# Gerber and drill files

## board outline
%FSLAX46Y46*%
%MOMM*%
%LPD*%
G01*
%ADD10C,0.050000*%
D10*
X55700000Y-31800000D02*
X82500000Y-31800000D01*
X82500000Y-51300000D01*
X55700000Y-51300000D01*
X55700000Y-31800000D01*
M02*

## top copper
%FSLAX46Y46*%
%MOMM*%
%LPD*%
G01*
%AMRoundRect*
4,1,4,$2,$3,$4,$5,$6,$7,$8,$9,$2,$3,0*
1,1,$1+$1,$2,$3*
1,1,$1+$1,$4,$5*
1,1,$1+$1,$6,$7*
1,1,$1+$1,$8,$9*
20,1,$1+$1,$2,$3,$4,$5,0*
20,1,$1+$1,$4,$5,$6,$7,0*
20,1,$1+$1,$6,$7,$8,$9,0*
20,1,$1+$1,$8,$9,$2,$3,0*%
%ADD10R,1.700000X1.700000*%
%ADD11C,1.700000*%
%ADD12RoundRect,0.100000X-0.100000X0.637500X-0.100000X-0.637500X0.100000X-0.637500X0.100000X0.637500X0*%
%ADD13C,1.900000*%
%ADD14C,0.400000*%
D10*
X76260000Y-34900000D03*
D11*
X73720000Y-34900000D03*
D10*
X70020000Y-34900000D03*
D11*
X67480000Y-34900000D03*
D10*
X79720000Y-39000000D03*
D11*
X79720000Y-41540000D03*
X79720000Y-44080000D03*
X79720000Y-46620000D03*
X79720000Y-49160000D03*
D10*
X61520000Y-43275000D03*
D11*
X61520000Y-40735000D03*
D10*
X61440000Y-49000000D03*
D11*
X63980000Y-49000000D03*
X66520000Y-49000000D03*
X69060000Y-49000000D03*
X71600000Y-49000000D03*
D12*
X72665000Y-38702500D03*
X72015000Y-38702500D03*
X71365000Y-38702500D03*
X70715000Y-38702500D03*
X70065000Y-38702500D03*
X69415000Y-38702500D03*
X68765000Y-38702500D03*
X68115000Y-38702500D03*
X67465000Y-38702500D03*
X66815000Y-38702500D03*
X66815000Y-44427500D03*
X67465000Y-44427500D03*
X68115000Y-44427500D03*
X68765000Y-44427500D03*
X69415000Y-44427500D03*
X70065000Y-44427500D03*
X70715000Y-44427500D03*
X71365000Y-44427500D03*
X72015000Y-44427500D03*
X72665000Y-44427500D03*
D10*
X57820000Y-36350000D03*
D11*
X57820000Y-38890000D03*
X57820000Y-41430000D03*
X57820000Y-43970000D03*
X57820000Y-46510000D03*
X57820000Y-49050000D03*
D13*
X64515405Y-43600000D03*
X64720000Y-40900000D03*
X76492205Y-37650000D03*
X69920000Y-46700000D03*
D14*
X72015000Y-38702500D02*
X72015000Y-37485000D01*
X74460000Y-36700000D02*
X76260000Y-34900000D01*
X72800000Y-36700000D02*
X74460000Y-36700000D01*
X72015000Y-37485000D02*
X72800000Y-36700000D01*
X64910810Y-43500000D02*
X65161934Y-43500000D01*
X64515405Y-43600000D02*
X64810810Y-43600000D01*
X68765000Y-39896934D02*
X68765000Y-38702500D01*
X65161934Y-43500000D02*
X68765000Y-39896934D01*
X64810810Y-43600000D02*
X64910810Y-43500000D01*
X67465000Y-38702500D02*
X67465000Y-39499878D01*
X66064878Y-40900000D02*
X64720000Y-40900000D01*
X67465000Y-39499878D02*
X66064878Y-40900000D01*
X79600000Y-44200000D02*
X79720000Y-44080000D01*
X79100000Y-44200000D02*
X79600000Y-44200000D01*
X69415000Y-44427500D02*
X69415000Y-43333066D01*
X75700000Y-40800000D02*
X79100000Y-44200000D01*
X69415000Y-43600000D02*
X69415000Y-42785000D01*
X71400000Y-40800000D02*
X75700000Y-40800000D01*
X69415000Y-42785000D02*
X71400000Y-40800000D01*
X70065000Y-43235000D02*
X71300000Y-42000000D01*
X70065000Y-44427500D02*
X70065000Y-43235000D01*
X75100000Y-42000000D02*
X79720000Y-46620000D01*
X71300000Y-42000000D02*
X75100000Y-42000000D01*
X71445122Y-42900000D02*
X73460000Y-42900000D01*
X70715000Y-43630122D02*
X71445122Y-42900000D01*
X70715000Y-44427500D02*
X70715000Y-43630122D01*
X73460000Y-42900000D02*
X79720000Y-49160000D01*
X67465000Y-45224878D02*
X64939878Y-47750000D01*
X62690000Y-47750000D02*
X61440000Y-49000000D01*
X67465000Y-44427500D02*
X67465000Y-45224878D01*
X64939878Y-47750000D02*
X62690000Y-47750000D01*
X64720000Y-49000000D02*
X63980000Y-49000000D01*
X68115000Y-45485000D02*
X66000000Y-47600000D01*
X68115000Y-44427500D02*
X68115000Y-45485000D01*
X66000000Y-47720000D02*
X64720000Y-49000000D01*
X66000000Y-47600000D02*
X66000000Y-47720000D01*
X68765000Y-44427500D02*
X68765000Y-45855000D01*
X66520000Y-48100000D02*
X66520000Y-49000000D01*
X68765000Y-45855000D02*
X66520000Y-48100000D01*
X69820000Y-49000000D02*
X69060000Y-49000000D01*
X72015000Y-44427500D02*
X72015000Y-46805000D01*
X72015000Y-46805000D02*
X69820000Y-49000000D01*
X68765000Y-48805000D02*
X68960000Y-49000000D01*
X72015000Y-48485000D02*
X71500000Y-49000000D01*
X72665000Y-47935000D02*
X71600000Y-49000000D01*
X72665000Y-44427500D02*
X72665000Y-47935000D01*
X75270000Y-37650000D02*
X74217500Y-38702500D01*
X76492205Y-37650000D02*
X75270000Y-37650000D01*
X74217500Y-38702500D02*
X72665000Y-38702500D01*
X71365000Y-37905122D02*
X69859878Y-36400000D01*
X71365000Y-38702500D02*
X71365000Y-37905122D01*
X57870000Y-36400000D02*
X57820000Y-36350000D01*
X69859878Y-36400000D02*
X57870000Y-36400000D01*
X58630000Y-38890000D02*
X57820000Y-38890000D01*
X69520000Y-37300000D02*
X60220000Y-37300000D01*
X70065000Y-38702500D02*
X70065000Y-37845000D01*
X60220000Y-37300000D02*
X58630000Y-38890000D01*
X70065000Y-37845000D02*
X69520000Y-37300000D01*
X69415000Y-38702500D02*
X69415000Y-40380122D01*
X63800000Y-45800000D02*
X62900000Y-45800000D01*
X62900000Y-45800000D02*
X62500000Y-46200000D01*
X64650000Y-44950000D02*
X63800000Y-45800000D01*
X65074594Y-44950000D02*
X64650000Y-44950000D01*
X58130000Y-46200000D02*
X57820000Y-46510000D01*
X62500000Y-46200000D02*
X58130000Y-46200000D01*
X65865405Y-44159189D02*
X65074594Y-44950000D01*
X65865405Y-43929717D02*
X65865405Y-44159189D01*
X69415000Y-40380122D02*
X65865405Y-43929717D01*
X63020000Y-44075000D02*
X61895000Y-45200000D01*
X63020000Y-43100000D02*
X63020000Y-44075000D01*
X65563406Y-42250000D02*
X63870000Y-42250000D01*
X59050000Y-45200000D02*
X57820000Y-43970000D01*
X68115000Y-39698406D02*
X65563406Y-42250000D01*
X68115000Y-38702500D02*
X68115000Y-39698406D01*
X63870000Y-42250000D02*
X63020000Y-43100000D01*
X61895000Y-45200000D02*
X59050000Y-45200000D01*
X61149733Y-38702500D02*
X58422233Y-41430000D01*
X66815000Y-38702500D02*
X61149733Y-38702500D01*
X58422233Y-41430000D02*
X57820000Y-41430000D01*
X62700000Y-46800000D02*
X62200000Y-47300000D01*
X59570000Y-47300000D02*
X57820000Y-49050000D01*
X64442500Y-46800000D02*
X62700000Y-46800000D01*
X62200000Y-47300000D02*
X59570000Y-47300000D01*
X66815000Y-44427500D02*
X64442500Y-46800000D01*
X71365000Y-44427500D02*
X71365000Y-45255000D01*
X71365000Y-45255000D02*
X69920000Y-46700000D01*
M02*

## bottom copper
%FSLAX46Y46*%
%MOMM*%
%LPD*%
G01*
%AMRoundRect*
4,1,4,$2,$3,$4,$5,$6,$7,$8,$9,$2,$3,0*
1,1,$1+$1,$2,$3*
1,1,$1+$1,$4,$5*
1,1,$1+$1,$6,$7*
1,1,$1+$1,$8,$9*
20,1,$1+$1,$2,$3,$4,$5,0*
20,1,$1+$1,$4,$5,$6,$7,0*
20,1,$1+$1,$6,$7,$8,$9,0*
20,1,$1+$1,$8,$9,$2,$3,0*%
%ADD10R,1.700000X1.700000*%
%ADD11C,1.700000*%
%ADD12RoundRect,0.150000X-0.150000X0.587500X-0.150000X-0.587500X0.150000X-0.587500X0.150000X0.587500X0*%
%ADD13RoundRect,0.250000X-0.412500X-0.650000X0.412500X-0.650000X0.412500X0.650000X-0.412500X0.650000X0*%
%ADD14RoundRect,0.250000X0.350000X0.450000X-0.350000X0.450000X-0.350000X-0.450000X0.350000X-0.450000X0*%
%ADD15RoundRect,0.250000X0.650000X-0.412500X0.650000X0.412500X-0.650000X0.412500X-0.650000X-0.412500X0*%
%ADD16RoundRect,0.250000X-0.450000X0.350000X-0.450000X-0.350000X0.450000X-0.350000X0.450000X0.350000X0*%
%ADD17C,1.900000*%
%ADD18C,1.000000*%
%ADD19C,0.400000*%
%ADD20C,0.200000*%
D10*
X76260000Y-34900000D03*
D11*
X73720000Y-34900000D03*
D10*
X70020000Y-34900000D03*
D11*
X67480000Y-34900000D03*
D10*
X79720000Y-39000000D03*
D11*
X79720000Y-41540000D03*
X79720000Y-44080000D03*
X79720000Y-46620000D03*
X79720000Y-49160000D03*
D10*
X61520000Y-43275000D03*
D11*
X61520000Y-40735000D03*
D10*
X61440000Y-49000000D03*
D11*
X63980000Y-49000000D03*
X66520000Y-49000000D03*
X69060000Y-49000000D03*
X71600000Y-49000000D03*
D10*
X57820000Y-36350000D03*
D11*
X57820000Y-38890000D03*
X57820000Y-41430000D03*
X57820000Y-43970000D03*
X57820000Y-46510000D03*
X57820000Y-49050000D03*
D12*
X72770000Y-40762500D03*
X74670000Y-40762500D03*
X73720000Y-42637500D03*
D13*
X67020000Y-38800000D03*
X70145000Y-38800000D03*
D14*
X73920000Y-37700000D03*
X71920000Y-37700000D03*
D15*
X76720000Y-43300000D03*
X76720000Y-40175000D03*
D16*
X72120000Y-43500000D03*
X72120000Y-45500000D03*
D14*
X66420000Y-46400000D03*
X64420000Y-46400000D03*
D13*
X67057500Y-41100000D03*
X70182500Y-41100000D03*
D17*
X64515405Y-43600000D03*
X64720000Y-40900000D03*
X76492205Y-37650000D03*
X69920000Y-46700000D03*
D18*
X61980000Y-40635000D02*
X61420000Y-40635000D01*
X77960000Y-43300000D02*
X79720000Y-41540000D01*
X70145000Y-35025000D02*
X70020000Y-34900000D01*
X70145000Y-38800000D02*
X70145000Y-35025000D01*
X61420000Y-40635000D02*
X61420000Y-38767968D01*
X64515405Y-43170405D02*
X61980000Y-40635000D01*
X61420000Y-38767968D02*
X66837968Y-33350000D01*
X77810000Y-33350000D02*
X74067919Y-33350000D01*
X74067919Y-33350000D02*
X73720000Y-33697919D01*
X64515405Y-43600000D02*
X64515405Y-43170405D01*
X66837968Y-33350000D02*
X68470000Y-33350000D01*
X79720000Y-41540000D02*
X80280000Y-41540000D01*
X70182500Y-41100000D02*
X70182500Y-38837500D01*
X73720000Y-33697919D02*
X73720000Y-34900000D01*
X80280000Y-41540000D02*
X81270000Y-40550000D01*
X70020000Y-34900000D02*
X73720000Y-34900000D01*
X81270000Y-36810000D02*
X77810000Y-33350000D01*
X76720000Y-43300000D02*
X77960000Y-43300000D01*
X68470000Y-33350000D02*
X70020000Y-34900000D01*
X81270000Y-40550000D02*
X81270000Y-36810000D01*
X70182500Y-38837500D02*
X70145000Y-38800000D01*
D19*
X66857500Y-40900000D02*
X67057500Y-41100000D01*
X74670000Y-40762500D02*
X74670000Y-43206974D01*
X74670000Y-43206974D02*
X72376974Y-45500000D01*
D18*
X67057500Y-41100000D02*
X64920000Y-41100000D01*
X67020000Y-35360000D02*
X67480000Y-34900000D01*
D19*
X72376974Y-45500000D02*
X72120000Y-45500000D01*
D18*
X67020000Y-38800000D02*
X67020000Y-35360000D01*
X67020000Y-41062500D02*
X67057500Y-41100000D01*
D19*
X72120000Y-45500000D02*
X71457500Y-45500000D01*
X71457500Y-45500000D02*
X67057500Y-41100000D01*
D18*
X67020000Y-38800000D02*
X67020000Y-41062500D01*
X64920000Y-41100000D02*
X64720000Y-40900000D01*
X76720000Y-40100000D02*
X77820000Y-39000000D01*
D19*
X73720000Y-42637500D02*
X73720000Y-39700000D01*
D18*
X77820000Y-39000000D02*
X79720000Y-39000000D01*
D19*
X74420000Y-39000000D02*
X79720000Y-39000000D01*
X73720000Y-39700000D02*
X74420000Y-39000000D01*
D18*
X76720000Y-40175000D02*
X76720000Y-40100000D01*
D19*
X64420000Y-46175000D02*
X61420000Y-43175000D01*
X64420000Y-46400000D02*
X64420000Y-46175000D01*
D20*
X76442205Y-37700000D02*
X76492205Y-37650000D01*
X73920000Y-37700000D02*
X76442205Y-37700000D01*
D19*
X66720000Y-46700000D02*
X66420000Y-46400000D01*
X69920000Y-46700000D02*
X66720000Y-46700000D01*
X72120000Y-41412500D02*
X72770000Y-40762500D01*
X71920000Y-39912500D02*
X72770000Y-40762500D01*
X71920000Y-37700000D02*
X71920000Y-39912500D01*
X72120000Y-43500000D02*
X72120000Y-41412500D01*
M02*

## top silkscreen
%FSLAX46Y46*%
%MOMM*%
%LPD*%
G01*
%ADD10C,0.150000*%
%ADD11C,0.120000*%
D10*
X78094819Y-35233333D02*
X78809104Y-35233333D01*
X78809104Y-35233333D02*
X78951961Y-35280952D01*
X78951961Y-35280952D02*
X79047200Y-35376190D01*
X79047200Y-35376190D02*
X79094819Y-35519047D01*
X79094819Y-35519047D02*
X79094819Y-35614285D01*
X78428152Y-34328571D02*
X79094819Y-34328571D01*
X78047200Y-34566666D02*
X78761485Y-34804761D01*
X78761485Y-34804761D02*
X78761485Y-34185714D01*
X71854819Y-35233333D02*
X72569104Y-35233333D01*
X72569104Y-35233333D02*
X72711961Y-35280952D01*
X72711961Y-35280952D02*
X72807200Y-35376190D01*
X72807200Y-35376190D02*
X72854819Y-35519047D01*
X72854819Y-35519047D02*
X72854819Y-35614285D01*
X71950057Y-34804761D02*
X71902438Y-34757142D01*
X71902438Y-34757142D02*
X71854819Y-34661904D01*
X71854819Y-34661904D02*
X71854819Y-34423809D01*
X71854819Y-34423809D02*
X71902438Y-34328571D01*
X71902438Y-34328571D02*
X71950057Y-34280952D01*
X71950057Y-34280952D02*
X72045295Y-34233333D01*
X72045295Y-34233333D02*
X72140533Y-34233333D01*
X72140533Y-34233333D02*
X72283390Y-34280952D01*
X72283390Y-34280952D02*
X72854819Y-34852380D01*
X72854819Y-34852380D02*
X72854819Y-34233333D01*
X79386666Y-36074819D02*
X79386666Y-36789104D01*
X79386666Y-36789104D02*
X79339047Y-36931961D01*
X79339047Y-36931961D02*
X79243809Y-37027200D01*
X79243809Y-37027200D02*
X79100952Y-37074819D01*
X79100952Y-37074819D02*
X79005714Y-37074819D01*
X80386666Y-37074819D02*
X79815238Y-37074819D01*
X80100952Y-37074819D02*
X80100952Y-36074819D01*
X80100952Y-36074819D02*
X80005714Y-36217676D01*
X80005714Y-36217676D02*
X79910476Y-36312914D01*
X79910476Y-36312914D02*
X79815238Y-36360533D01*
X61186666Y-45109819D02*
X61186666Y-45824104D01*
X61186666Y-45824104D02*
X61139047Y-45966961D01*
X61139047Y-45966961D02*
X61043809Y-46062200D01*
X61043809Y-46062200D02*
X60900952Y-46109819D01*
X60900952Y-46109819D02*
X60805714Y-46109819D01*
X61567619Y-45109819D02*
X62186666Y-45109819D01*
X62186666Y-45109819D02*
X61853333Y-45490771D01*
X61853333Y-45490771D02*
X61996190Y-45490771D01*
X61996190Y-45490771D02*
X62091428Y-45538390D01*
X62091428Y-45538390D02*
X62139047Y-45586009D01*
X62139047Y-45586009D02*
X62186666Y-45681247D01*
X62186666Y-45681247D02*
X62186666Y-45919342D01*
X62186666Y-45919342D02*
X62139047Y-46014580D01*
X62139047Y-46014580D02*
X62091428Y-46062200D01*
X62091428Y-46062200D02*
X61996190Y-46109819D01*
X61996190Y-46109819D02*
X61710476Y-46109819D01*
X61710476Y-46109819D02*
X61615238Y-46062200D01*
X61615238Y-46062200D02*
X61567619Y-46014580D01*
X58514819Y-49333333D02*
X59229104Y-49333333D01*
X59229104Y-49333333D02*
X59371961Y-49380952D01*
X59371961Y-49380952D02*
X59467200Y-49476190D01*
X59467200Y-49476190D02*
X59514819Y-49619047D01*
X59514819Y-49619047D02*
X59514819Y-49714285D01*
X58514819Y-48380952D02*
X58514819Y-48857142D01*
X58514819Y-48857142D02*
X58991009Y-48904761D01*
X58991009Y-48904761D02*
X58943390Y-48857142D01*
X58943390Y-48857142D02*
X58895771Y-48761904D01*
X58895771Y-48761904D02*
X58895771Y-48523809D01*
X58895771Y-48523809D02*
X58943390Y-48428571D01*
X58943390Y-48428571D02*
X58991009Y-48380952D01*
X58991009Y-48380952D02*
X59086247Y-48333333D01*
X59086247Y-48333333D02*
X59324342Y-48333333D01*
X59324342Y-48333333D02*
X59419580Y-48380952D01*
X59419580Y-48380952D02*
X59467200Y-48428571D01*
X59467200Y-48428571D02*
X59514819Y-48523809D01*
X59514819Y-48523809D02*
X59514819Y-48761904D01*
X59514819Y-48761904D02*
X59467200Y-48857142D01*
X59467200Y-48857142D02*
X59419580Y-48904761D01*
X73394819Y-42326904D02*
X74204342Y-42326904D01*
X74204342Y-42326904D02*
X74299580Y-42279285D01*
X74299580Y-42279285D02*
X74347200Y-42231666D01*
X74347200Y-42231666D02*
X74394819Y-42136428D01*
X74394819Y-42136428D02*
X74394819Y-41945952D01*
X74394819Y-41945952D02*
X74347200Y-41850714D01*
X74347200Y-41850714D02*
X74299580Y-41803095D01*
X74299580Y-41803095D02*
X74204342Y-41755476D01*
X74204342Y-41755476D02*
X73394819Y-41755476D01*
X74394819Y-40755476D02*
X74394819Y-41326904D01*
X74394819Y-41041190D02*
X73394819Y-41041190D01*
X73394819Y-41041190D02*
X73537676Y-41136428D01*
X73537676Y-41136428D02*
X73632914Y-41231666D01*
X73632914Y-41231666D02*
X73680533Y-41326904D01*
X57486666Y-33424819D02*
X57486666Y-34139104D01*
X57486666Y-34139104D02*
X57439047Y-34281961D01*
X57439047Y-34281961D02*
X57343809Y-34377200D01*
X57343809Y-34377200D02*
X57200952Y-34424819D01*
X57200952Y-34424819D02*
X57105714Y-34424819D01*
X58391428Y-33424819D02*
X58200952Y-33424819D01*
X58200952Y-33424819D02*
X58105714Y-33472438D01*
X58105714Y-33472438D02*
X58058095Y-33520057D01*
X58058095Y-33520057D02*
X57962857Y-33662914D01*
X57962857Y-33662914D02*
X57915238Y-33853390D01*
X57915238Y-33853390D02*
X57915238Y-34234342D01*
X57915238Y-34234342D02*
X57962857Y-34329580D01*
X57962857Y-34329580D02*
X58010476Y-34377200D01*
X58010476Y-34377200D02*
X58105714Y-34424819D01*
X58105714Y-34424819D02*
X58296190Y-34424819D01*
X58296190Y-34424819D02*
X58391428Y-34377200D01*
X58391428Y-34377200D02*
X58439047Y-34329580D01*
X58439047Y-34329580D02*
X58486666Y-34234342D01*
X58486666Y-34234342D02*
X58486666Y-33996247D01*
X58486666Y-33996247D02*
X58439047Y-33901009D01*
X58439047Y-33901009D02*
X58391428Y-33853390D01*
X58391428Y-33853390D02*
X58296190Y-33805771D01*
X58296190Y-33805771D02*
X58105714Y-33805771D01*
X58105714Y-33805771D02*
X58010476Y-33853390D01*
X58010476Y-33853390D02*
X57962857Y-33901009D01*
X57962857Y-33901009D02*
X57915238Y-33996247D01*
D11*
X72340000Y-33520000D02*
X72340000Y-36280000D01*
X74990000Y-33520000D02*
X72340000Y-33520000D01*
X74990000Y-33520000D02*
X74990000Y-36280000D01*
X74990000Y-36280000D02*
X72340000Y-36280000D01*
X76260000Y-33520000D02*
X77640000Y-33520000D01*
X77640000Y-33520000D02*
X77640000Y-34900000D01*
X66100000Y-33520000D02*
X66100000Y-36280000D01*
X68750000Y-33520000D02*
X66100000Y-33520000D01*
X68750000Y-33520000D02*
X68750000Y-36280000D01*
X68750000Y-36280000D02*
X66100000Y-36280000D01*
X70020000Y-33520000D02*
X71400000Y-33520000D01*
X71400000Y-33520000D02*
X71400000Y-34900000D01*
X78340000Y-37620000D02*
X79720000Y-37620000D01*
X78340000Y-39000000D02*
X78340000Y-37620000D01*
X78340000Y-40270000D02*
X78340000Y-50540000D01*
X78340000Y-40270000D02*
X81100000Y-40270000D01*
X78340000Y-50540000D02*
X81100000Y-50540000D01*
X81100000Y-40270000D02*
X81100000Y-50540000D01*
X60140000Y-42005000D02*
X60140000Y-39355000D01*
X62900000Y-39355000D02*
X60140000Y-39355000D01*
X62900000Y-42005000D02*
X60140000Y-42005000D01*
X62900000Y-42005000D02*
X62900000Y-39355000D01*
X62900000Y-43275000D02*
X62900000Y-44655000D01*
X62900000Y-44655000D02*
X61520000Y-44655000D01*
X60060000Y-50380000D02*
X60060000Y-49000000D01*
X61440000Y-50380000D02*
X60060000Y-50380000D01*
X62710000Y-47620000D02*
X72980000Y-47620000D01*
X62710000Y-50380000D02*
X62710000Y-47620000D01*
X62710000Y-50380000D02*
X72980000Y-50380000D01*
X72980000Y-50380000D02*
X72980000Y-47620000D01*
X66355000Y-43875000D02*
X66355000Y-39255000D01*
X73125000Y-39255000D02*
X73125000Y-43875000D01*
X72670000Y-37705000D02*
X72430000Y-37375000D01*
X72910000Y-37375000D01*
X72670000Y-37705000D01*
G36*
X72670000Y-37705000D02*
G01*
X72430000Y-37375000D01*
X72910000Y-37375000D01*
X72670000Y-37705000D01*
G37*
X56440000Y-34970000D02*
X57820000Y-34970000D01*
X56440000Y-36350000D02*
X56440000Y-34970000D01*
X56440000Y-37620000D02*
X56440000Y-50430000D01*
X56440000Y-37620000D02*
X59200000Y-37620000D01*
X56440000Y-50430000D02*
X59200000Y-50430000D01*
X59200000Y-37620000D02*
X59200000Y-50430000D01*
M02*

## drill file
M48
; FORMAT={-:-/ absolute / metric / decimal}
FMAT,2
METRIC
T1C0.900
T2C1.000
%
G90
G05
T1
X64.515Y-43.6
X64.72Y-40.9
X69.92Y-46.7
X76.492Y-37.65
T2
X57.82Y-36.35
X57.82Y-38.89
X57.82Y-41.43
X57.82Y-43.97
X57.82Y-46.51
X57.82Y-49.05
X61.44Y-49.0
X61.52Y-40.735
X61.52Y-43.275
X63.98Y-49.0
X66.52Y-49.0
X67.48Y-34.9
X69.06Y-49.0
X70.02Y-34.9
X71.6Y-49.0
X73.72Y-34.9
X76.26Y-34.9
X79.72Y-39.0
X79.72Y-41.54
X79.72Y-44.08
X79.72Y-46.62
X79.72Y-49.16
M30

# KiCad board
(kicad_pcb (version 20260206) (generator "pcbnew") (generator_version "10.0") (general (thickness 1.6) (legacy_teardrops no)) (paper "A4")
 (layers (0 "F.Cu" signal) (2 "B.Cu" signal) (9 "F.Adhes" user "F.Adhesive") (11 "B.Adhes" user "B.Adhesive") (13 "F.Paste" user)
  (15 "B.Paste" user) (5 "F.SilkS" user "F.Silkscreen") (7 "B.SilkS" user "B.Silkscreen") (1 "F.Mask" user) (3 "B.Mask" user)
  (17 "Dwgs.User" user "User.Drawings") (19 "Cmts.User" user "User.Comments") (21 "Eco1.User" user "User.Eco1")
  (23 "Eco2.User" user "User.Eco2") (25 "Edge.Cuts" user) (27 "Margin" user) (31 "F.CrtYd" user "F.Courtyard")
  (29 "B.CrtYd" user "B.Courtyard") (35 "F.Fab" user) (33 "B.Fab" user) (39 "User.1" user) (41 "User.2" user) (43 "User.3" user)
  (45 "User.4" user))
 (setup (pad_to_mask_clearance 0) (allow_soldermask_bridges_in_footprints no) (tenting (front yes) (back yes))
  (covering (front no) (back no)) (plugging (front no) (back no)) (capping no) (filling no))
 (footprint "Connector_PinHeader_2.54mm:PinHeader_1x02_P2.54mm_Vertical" (layer "F.Cu") (at 76.26 34.9 -90)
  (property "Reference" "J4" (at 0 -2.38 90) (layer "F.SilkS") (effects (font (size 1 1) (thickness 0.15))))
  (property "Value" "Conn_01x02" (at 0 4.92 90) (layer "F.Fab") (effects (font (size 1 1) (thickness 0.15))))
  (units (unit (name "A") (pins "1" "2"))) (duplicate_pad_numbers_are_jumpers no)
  (fp_line (start -1.38 3.92) (end 1.38 3.92) (stroke (width 0.12) (type solid)) (layer "F.SilkS"))
  (fp_line (start -1.38 1.27) (end -1.38 3.92) (stroke (width 0.12) (type solid)) (layer "F.SilkS"))
  (fp_line (start -1.38 1.27) (end 1.38 1.27) (stroke (width 0.12) (type solid)) (layer "F.SilkS"))
  (fp_line (start 1.38 1.27) (end 1.38 3.92) (stroke (width 0.12) (type solid)) (layer "F.SilkS"))
  (fp_line (start -1.38 0) (end -1.38 -1.38) (stroke (width 0.12) (type solid)) (layer "F.SilkS"))
  (fp_line (start -1.38 -1.38) (end 0 -1.38) (stroke (width 0.12) (type solid)) (layer "F.SilkS"))
  (pad "1" thru_hole rect (at 0 0 270) (size 1.7 1.7) (drill 1) (layers "*.Cu" "*.Mask") (remove_unused_layers no) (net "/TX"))
  (pad "2" thru_hole circle (at 0 2.54 270) (size 1.7 1.7) (drill 1) (layers "*.Cu" "*.Mask") (remove_unused_layers no) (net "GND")))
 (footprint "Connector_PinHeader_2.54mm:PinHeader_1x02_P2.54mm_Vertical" (layer "F.Cu") (at 70.02 34.9 -90)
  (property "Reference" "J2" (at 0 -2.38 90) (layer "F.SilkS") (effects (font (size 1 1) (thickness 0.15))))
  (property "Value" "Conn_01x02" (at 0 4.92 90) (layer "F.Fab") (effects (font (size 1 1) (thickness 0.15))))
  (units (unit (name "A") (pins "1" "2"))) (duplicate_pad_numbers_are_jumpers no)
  (fp_line (start -1.38 3.92) (end 1.38 3.92) (stroke (width 0.12) (type solid)) (layer "F.SilkS"))
  (fp_line (start -1.38 1.27) (end -1.38 3.92) (stroke (width 0.12) (type solid)) (layer "F.SilkS"))
  (fp_line (start -1.38 1.27) (end 1.38 1.27) (stroke (width 0.12) (type solid)) (layer "F.SilkS"))
  (fp_line (start 1.38 1.27) (end 1.38 3.92) (stroke (width 0.12) (type solid)) (layer "F.SilkS"))
  (fp_line (start -1.38 0) (end -1.38 -1.38) (stroke (width 0.12) (type solid)) (layer "F.SilkS"))
  (fp_line (start -1.38 -1.38) (end 0 -1.38) (stroke (width 0.12) (type solid)) (layer "F.SilkS"))
  (pad "1" thru_hole rect (at 0 0 270) (size 1.7 1.7) (drill 1) (layers "*.Cu" "*.Mask") (remove_unused_layers no) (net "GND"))
  (pad "2" thru_hole circle (at 0 2.54 270) (size 1.7 1.7) (drill 1) (layers "*.Cu" "*.Mask") (remove_unused_layers no) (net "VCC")))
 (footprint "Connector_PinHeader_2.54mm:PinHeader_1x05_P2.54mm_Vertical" (layer "F.Cu") (at 79.72 39)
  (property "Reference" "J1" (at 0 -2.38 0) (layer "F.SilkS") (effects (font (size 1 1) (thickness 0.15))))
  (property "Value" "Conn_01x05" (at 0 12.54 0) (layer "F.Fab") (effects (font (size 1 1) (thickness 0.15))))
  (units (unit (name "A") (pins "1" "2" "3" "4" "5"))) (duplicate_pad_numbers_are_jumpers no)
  (fp_line (start -1.38 -1.38) (end 0 -1.38) (stroke (width 0.12) (type solid)) (layer "F.SilkS"))
  (fp_line (start -1.38 0) (end -1.38 -1.38) (stroke (width 0.12) (type solid)) (layer "F.SilkS"))
  (fp_line (start -1.38 1.27) (end -1.38 11.54) (stroke (width 0.12) (type solid)) (layer "F.SilkS"))
  (fp_line (start -1.38 1.27) (end 1.38 1.27) (stroke (width 0.12) (type solid)) (layer "F.SilkS"))
  (fp_line (start -1.38 11.54) (end 1.38 11.54) (stroke (width 0.12) (type solid)) (layer "F.SilkS"))
  (fp_line (start 1.38 1.27) (end 1.38 11.54) (stroke (width 0.12) (type solid)) (layer "F.SilkS"))
  (pad "1" thru_hole rect (at 0 0) (size 1.7 1.7) (drill 1) (layers "*.Cu" "*.Mask") (remove_unused_layers no) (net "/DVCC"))
  (pad "2" thru_hole circle (at 0 2.54) (size 1.7 1.7) (drill 1) (layers "*.Cu" "*.Mask") (remove_unused_layers no) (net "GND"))
  (pad "3" thru_hole circle (at 0 5.08) (size 1.7 1.7) (drill 1) (layers "*.Cu" "*.Mask") (remove_unused_layers no) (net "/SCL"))
  (pad "4" thru_hole circle (at 0 7.62) (size 1.7 1.7) (drill 1) (layers "*.Cu" "*.Mask") (remove_unused_layers no) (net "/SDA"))
  (pad "5" thru_hole circle (at 0 10.16) (size 1.7 1.7) (drill 1) (layers "*.Cu" "*.Mask") (remove_unused_layers no) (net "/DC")))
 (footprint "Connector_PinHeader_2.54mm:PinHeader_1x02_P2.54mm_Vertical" (layer "F.Cu") (at 61.52 43.275 180)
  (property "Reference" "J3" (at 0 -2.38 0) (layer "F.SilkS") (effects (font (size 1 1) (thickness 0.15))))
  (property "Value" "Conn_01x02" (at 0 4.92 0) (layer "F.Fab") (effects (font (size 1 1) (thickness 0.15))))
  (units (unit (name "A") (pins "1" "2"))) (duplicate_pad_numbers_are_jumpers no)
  (fp_line (start 1.38 1.27) (end 1.38 3.92) (stroke (width 0.12) (type solid)) (layer "F.SilkS"))
  (fp_line (start -1.38 3.92) (end 1.38 3.92) (stroke (width 0.12) (type solid)) (layer "F.SilkS"))
  (fp_line (start -1.38 1.27) (end 1.38 1.27) (stroke (width 0.12) (type solid)) (layer "F.SilkS"))
  (fp_line (start -1.38 1.27) (end -1.38 3.92) (stroke (width 0.12) (type solid)) (layer "F.SilkS"))
  (fp_line (start -1.38 0) (end -1.38 -1.38) (stroke (width 0.12) (type solid)) (layer "F.SilkS"))
  (fp_line (start -1.38 -1.38) (end 0 -1.38) (stroke (width 0.12) (type solid)) (layer "F.SilkS"))
  (pad "1" thru_hole rect (at 0 0 180) (size 1.7 1.7) (drill 1) (layers "*.Cu" "*.Mask") (remove_unused_layers no) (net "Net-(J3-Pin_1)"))
  (pad "2" thru_hole circle (at 0 2.54 180) (size 1.7 1.7) (drill 1) (layers "*.Cu" "*.Mask") (remove_unused_layers no) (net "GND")))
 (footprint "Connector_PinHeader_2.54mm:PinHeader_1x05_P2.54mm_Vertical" (layer "F.Cu") (at 61.44 49 90)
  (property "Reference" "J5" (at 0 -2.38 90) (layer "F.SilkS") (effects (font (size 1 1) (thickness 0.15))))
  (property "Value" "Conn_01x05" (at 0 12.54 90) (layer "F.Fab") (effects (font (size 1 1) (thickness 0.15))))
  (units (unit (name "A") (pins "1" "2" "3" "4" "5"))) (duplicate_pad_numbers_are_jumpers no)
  (fp_line (start -1.38 -1.38) (end 0 -1.38) (stroke (width 0.12) (type solid)) (layer "F.SilkS"))
  (fp_line (start -1.38 0) (end -1.38 -1.38) (stroke (width 0.12) (type solid)) (layer "F.SilkS"))
  (fp_line (start 1.38 1.27) (end 1.38 11.54) (stroke (width 0.12) (type solid)) (layer "F.SilkS"))
  (fp_line (start -1.38 1.27) (end 1.38 1.27) (stroke (width 0.12) (type solid)) (layer "F.SilkS"))
  (fp_line (start -1.38 1.27) (end -1.38 11.54) (stroke (width 0.12) (type solid)) (layer "F.SilkS"))
  (fp_line (start -1.38 11.54) (end 1.38 11.54) (stroke (width 0.12) (type solid)) (layer "F.SilkS"))
  (pad "1" thru_hole rect (at 0 0 90) (size 1.7 1.7) (drill 1) (layers "*.Cu" "*.Mask") (remove_unused_layers no) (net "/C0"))
  (pad "2" thru_hole circle (at 0 2.54 90) (size 1.7 1.7) (drill 1) (layers "*.Cu" "*.Mask") (remove_unused_layers no) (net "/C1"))
  (pad "3" thru_hole circle (at 0 5.08 90) (size 1.7 1.7) (drill 1) (layers "*.Cu" "*.Mask") (remove_unused_layers no) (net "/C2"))
  (pad "4" thru_hole circle (at 0 7.62 90) (size 1.7 1.7) (drill 1) (layers "*.Cu" "*.Mask") (remove_unused_layers no) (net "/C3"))
  (pad "5" thru_hole circle (at 0 10.16 90) (size 1.7 1.7) (drill 1) (layers "*.Cu" "*.Mask") (remove_unused_layers no) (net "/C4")))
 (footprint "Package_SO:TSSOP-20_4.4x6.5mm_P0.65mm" (layer "F.Cu") (at 69.74 41.565 -90)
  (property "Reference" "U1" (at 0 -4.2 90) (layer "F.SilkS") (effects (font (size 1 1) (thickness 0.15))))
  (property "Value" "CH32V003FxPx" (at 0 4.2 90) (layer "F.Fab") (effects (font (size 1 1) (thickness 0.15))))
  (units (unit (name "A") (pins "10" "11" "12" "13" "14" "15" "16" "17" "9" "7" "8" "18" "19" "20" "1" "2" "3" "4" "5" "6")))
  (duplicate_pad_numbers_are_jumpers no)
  (fp_line (start 2.31 3.385) (end -2.31 3.385) (stroke (width 0.12) (type solid)) (layer "F.SilkS"))
  (fp_line (start -2.31 -3.385) (end 2.31 -3.385) (stroke (width 0.12) (type solid)) (layer "F.SilkS"))
  (fp_poly (pts (xy -3.86 -2.93) (xy -4.19 -2.69) (xy -4.19 -3.17)) (stroke (width 0.12) (type solid)) (fill yes) (layer "F.SilkS"))
  (pad "1" smd roundrect (at -2.8625 -2.925 270) (size 1.475 0.4) (layers "F.Cu" "F.Mask" "F.Paste") (roundrect_rratio 0.25)
   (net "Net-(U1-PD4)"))
  (pad "2" smd roundrect (at -2.8625 -2.275 270) (size 1.475 0.4) (layers "F.Cu" "F.Mask" "F.Paste") (roundrect_rratio 0.25) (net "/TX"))
  (pad "3" smd roundrect (at -2.8625 -1.625 270) (size 1.475 0.4) (layers "F.Cu" "F.Mask" "F.Paste") (roundrect_rratio 0.25) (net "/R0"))
  (pad "4" smd roundrect (at -2.8625 -0.975 270) (size 1.475 0.4) (layers "F.Cu" "F.Mask" "F.Paste") (roundrect_rratio 0.25) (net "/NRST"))
  (pad "5" smd roundrect (at -2.8625 -0.325 270) (size 1.475 0.4) (layers "F.Cu" "F.Mask" "F.Paste") (roundrect_rratio 0.25) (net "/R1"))
  (pad "6" smd roundrect (at -2.8625 0.325 270) (size 1.475 0.4) (layers "F.Cu" "F.Mask" "F.Paste") (roundrect_rratio 0.25) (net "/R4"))
  (pad "7" smd roundrect (at -2.8625 0.975 270) (size 1.475 0.4) (layers "F.Cu" "F.Mask" "F.Paste") (roundrect_rratio 0.25) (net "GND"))
  (pad "8" smd roundrect (at -2.8625 1.625 270) (size 1.475 0.4) (layers "F.Cu" "F.Mask" "F.Paste") (roundrect_rratio 0.25) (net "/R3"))
  (pad "9" smd roundrect (at -2.8625 2.275 270) (size 1.475 0.4) (layers "F.Cu" "F.Mask" "F.Paste") (roundrect_rratio 0.25) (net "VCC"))
  (pad "10" smd roundrect (at -2.8625 2.925 270) (size 1.475 0.4) (layers "F.Cu" "F.Mask" "F.Paste") (roundrect_rratio 0.25) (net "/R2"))
  (pad "11" smd roundrect (at 2.8625 2.925 270) (size 1.475 0.4) (layers "F.Cu" "F.Mask" "F.Paste") (roundrect_rratio 0.25) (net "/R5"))
  (pad "12" smd roundrect (at 2.8625 2.275 270) (size 1.475 0.4) (layers "F.Cu" "F.Mask" "F.Paste") (roundrect_rratio 0.25) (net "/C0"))
  (pad "13" smd roundrect (at 2.8625 1.625 270) (size 1.475 0.4) (layers "F.Cu" "F.Mask" "F.Paste") (roundrect_rratio 0.25) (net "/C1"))
  (pad "14" smd roundrect (at 2.8625 0.975 270) (size 1.475 0.4) (layers "F.Cu" "F.Mask" "F.Paste") (roundrect_rratio 0.25) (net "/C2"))
  (pad "15" smd roundrect (at 2.8625 0.325 270) (size 1.475 0.4) (layers "F.Cu" "F.Mask" "F.Paste") (roundrect_rratio 0.25) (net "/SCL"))
  (pad "16" smd roundrect (at 2.8625 -0.325 270) (size 1.475 0.4) (layers "F.Cu" "F.Mask" "F.Paste") (roundrect_rratio 0.25) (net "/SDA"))
  (pad "17" smd roundrect (at 2.8625 -0.975 270) (size 1.475 0.4) (layers "F.Cu" "F.Mask" "F.Paste") (roundrect_rratio 0.25) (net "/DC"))
  (pad "18" smd roundrect (at 2.8625 -1.625 270) (size 1.475 0.4) (layers "F.Cu" "F.Mask" "F.Paste") (roundrect_rratio 0.25) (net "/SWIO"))
  (pad "19" smd roundrect (at 2.8625 -2.275 270) (size 1.475 0.4) (layers "F.Cu" "F.Mask" "F.Paste") (roundrect_rratio 0.25) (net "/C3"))
  (pad "20" smd roundrect (at 2.8625 -2.925 270) (size 1.475 0.4) (layers "F.Cu" "F.Mask" "F.Paste") (roundrect_rratio 0.25) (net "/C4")))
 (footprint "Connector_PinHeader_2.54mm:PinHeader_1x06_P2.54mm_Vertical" (layer "F.Cu") (at 57.82 36.35)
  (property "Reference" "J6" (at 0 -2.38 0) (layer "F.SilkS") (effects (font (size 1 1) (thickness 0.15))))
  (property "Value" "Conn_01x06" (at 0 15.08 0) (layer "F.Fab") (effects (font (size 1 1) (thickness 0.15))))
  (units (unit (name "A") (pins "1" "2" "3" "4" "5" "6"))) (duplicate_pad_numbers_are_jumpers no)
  (fp_line (start -1.38 -1.38) (end 0 -1.38) (stroke (width 0.12) (type solid)) (layer "F.SilkS"))
  (fp_line (start -1.38 0) (end -1.38 -1.38) (stroke (width 0.12) (type solid)) (layer "F.SilkS"))
  (fp_line (start -1.38 1.27) (end -1.38 14.08) (stroke (width 0.12) (type solid)) (layer "F.SilkS"))
  (fp_line (start -1.38 1.27) (end 1.38 1.27) (stroke (width 0.12) (type solid)) (layer "F.SilkS"))
  (fp_line (start -1.38 14.08) (end 1.38 14.08) (stroke (width 0.12) (type solid)) (layer "F.SilkS"))
  (fp_line (start 1.38 1.27) (end 1.38 14.08) (stroke (width 0.12) (type solid)) (layer "F.SilkS"))
  (pad "1" thru_hole rect (at 0 0) (size 1.7 1.7) (drill 1) (layers "*.Cu" "*.Mask") (remove_unused_layers no) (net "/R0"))
  (pad "2" thru_hole circle (at 0 2.54) (size 1.7 1.7) (drill 1) (layers "*.Cu" "*.Mask") (remove_unused_layers no) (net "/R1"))
  (pad "3" thru_hole circle (at 0 5.08) (size 1.7 1.7) (drill 1) (layers "*.Cu" "*.Mask") (remove_unused_layers no) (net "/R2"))
  (pad "4" thru_hole circle (at 0 7.62) (size 1.7 1.7) (drill 1) (layers "*.Cu" "*.Mask") (remove_unused_layers no) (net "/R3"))
  (pad "5" thru_hole circle (at 0 10.16) (size 1.7 1.7) (drill 1) (layers "*.Cu" "*.Mask") (remove_unused_layers no) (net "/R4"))
  (pad "6" thru_hole circle (at 0 12.7) (size 1.7 1.7) (drill 1) (layers "*.Cu" "*.Mask") (remove_unused_layers no) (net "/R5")))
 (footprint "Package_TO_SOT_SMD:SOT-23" (layer "B.Cu") (at 73.72 41.7 -90)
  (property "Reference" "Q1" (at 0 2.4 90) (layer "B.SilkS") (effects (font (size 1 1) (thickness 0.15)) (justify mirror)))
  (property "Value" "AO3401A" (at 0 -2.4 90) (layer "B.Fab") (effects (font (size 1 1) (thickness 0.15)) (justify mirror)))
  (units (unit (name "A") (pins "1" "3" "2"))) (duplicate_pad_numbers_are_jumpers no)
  (pad "1" smd roundrect (at -0.9375 0.95 270) (size 1.475 0.6) (layers "B.Cu" "B.Mask" "B.Paste") (roundrect_rratio 0.25)
   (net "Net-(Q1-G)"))
  (pad "2" smd roundrect (at -0.9375 -0.95 270) (size 1.475 0.6) (layers "B.Cu" "B.Mask" "B.Paste") (roundrect_rratio 0.25) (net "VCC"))
  (pad "3" smd roundrect (at 0.9375 0 270) (size 1.475 0.6) (layers "B.Cu" "B.Mask" "B.Paste") (roundrect_rratio 0.25) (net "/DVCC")))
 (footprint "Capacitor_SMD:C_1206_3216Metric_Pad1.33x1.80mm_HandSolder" (layer "B.Cu") (at 68.5825 38.8)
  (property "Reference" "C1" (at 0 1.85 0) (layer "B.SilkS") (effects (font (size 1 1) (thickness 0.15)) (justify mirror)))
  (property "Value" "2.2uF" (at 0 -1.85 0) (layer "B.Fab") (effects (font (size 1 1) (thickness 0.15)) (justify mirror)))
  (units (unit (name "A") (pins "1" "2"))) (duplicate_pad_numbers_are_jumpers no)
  (pad "1" smd roundrect (at -1.5625 0) (size 1.325 1.8) (layers "B.Cu" "B.Mask" "B.Paste") (roundrect_rratio 0.188679) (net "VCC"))
  (pad "2" smd roundrect (at 1.5625 0) (size 1.325 1.8) (layers "B.Cu" "B.Mask" "B.Paste") (roundrect_rratio 0.188679) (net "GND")))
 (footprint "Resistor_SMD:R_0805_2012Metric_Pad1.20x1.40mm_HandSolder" (layer "B.Cu") (at 72.92 37.7 180)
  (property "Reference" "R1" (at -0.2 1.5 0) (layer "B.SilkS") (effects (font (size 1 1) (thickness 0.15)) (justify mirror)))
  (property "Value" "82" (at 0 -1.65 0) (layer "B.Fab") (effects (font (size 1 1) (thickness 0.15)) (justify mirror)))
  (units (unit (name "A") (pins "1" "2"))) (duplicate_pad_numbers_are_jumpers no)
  (pad "1" smd roundrect (at -1 0 180) (size 1.2 1.4) (layers "B.Cu" "B.Mask" "B.Paste") (roundrect_rratio 0.208333) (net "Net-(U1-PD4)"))
  (pad "2" smd roundrect (at 1 0 180) (size 1.2 1.4) (layers "B.Cu" "B.Mask" "B.Paste") (roundrect_rratio 0.208333) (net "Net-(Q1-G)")))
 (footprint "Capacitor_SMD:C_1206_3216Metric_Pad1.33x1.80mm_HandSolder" (layer "B.Cu") (at 76.72 41.7375 90)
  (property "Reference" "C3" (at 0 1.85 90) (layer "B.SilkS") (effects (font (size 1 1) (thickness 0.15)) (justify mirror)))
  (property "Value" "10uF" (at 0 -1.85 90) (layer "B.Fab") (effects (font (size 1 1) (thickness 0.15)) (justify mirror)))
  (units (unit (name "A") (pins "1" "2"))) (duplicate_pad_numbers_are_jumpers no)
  (pad "1" smd roundrect (at -1.5625 0 90) (size 1.325 1.8) (layers "B.Cu" "B.Mask" "B.Paste") (roundrect_rratio 0.188679) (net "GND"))
  (pad "2" smd roundrect (at 1.5625 0 90) (size 1.325 1.8) (layers "B.Cu" "B.Mask" "B.Paste") (roundrect_rratio 0.188679) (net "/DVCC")))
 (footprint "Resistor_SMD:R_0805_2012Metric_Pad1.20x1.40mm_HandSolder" (layer "B.Cu") (at 72.12 44.5 -90)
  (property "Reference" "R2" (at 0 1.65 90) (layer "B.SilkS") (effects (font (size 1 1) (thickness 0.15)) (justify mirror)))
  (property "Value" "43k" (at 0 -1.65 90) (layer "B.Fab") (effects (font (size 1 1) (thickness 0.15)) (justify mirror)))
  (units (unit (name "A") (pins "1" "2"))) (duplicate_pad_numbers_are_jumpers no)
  (pad "1" smd roundrect (at -1 0 270) (size 1.2 1.4) (layers "B.Cu" "B.Mask" "B.Paste") (roundrect_rratio 0.208333) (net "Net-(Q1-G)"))
  (pad "2" smd roundrect (at 1 0 270) (size 1.2 1.4) (layers "B.Cu" "B.Mask" "B.Paste") (roundrect_rratio 0.208333) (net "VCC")))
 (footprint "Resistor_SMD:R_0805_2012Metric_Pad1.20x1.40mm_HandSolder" (layer "B.Cu") (at 65.42 46.4 180)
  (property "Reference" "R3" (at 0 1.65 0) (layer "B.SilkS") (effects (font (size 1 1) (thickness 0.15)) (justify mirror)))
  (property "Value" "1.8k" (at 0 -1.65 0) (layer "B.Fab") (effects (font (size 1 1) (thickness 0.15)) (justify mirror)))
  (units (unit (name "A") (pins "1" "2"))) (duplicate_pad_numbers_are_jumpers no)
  (pad "1" smd roundrect (at -1 0 180) (size 1.2 1.4) (layers "B.Cu" "B.Mask" "B.Paste") (roundrect_rratio 0.208333) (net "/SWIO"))
  (pad "2" smd roundrect (at 1 0 180) (size 1.2 1.4) (layers "B.Cu" "B.Mask" "B.Paste") (roundrect_rratio 0.208333) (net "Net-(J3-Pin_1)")))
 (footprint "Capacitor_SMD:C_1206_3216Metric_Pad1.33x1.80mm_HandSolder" (layer "B.Cu") (at 68.62 41.1)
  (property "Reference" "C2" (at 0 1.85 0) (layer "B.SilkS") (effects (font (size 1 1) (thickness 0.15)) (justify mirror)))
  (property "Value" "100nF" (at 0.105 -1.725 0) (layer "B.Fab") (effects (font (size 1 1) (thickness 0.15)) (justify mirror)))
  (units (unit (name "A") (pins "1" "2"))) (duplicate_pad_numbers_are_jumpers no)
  (pad "1" smd roundrect (at -1.5625 0) (size 1.325 1.8) (layers "B.Cu" "B.Mask" "B.Paste") (roundrect_rratio 0.188679) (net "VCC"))
  (pad "2" smd roundrect (at 1.5625 0) (size 1.325 1.8) (layers "B.Cu" "B.Mask" "B.Paste") (roundrect_rratio 0.188679) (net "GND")))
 (gr_rect (start 55.7 31.8) (end 82.5 51.3) (stroke (width 0.05) (type default)) (fill no) (layer "Edge.Cuts"))
 (segment (start 72.015 38.7025) (end 72.015 37.485) (width 0.4) (layer "F.Cu") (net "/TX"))
 (segment (start 74.46 36.7) (end 76.26 34.9) (width 0.4) (layer "F.Cu") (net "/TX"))
 (segment (start 72.8 36.7) (end 74.46 36.7) (width 0.4) (layer "F.Cu") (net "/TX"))
 (segment (start 72.015 37.485) (end 72.8 36.7) (width 0.4) (layer "F.Cu") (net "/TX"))
 (segment (start 64.91081 43.5) (end 65.161934 43.5) (width 0.4) (layer "F.Cu") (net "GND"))
 (segment (start 64.515405 43.6) (end 64.81081 43.6) (width 0.4) (layer "F.Cu") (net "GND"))
 (segment (start 68.765 39.896934) (end 68.765 38.7025) (width 0.4) (layer "F.Cu") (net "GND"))
 (segment (start 65.161934 43.5) (end 68.765 39.896934) (width 0.4) (layer "F.Cu") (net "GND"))
 (segment (start 64.81081 43.6) (end 64.91081 43.5) (width 0.4) (layer "F.Cu") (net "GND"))
 (via (at 64.515405 43.6) (size 1.9) (drill 0.9) (layers "F.Cu" "B.Cu") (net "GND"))
 (segment (start 61.98 40.635) (end 61.42 40.635) (width 1) (layer "B.Cu") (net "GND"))
 (segment (start 77.96 43.3) (end 79.72 41.54) (width 1) (layer "B.Cu") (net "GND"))
 (segment (start 70.145 35.025) (end 70.02 34.9) (width 1) (layer "B.Cu") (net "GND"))
 (segment (start 70.145 38.8) (end 70.145 35.025) (width 1) (layer "B.Cu") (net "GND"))
 (segment (start 61.42 40.635) (end 61.42 38.767968) (width 1) (layer "B.Cu") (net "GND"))
 (segment (start 64.515405 43.170405) (end 61.98 40.635) (width 1) (layer "B.Cu") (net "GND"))
 (segment (start 61.42 38.767968) (end 66.837968 33.35) (width 1) (layer "B.Cu") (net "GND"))
 (segment (start 77.81 33.35) (end 74.067919 33.35) (width 1) (layer "B.Cu") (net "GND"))
 (segment (start 74.067919 33.35) (end 73.72 33.697919) (width 1) (layer "B.Cu") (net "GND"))
 (segment (start 64.515405 43.6) (end 64.515405 43.170405) (width 1) (layer "B.Cu") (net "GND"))
 (segment (start 66.837968 33.35) (end 68.47 33.35) (width 1) (layer "B.Cu") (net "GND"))
 (segment (start 79.72 41.54) (end 80.28 41.54) (width 1) (layer "B.Cu") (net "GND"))
 (segment (start 70.1825 41.1) (end 70.1825 38.8375) (width 1) (layer "B.Cu") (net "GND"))
 (segment (start 73.72 33.697919) (end 73.72 34.9) (width 1) (layer "B.Cu") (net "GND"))
 (segment (start 80.28 41.54) (end 81.27 40.55) (width 1) (layer "B.Cu") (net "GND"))
 (segment (start 70.02 34.9) (end 73.72 34.9) (width 1) (layer "B.Cu") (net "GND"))
 (segment (start 81.27 36.81) (end 77.81 33.35) (width 1) (layer "B.Cu") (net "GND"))
 (segment (start 76.72 43.3) (end 77.96 43.3) (width 1) (layer "B.Cu") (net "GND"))
 (segment (start 68.47 33.35) (end 70.02 34.9) (width 1) (layer "B.Cu") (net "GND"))
 (segment (start 81.27 40.55) (end 81.27 36.81) (width 1) (layer "B.Cu") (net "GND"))
 (segment (start 70.1825 38.8375) (end 70.145 38.8) (width 1) (layer "B.Cu") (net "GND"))
 (segment (start 67.465 38.7025) (end 67.465 39.499878) (width 0.4) (layer "F.Cu") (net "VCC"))
 (segment (start 66.064878 40.9) (end 64.72 40.9) (width 0.4) (layer "F.Cu") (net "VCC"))
 (segment (start 67.465 39.499878) (end 66.064878 40.9) (width 0.4) (layer "F.Cu") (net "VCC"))
 (via (at 64.72 40.9) (size 1.9) (drill 0.9) (layers "F.Cu" "B.Cu") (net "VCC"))
 (segment (start 66.8575 40.9) (end 67.0575 41.1) (width 0.4) (layer "B.Cu") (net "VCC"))
 (segment (start 74.67 40.7625) (end 74.67 43.206974) (width 0.4) (layer "B.Cu") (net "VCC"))
 (segment (start 74.67 43.206974) (end 72.376974 45.5) (width 0.4) (layer "B.Cu") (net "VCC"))
 (segment (start 67.0575 41.1) (end 64.92 41.1) (width 1) (layer "B.Cu") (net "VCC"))
 (segment (start 67.02 35.36) (end 67.48 34.9) (width 1) (layer "B.Cu") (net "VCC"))
 (segment (start 72.376974 45.5) (end 72.12 45.5) (width 0.4) (layer "B.Cu") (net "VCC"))
 (segment (start 67.02 38.8) (end 67.02 35.36) (width 1) (layer "B.Cu") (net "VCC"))
 (segment (start 67.02 41.0625) (end 67.0575 41.1) (width 1) (layer "B.Cu") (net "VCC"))
 (segment (start 72.12 45.5) (end 71.4575 45.5) (width 0.4) (layer "B.Cu") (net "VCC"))
 (segment (start 71.4575 45.5) (end 67.0575 41.1) (width 0.4) (layer "B.Cu") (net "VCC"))
 (segment (start 67.02 38.8) (end 67.02 41.0625) (width 1) (layer "B.Cu") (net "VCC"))
 (segment (start 64.92 41.1) (end 64.72 40.9) (width 1) (layer "B.Cu") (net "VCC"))
 (segment (start 76.72 40.1) (end 77.82 39) (width 1) (layer "B.Cu") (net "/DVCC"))
 (segment (start 73.72 42.6375) (end 73.72 39.7) (width 0.4) (layer "B.Cu") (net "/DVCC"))
 (segment (start 77.82 39) (end 79.72 39) (width 1) (layer "B.Cu") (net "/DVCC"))
 (segment (start 74.42 39) (end 79.72 39) (width 0.4) (layer "B.Cu") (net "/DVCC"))
 (segment (start 73.72 39.7) (end 74.42 39) (width 0.4) (layer "B.Cu") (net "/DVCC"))
 (segment (start 76.72 40.175) (end 76.72 40.1) (width 1) (layer "B.Cu") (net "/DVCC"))
 (segment (start 79.6 44.2) (end 79.72 44.08) (width 0.4) (layer "F.Cu") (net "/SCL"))
 (segment (start 79.1 44.2) (end 79.6 44.2) (width 0.4) (layer "F.Cu") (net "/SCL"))
 (segment (start 69.415 44.4275) (end 69.415 43.333066) (width 0.4) (layer "F.Cu") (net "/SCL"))
 (segment (start 75.7 40.8) (end 79.1 44.2) (width 0.4) (layer "F.Cu") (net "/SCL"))
 (segment (start 69.415 43.6) (end 69.415 42.785) (width 0.4) (layer "F.Cu") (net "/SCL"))
 (segment (start 71.4 40.8) (end 75.7 40.8) (width 0.4) (layer "F.Cu") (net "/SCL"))
 (segment (start 69.415 42.785) (end 71.4 40.8) (width 0.4) (layer "F.Cu") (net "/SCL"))
 (segment (start 70.065 43.235) (end 71.3 42) (width 0.4) (layer "F.Cu") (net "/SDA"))
 (segment (start 70.065 44.4275) (end 70.065 43.235) (width 0.4) (layer "F.Cu") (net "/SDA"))
 (segment (start 75.1 42) (end 79.72 46.62) (width 0.4) (layer "F.Cu") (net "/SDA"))
 (segment (start 71.3 42) (end 75.1 42) (width 0.4) (layer "F.Cu") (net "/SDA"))
 (segment (start 71.445122 42.9) (end 73.46 42.9) (width 0.4) (layer "F.Cu") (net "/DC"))
 (segment (start 70.715 43.630122) (end 71.445122 42.9) (width 0.4) (layer "F.Cu") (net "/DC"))
 (segment (start 70.715 44.4275) (end 70.715 43.630122) (width 0.4) (layer "F.Cu") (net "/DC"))
 (segment (start 73.46 42.9) (end 79.72 49.16) (width 0.4) (layer "F.Cu") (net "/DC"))
 (segment (start 64.42 46.175) (end 61.42 43.175) (width 0.4) (layer "B.Cu") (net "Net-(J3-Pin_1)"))
 (segment (start 64.42 46.4) (end 64.42 46.175) (width 0.4) (layer "B.Cu") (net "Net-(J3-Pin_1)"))
 (segment (start 67.465 45.224878) (end 64.939878 47.75) (width 0.4) (layer "F.Cu") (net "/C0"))
 (segment (start 62.69 47.75) (end 61.44 49) (width 0.4) (layer "F.Cu") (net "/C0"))
 (segment (start 67.465 44.4275) (end 67.465 45.224878) (width 0.4) (layer "F.Cu") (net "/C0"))
 (segment (start 64.939878 47.75) (end 62.69 47.75) (width 0.4) (layer "F.Cu") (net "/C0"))
 (segment (start 64.72 49) (end 63.98 49) (width 0.4) (layer "F.Cu") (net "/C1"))
 (segment (start 68.115 45.485) (end 66 47.6) (width 0.4) (layer "F.Cu") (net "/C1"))
 (segment (start 68.115 44.4275) (end 68.115 45.485) (width 0.4) (layer "F.Cu") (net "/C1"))
 (segment (start 66 47.72) (end 64.72 49) (width 0.4) (layer "F.Cu") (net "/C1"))
 (segment (start 66 47.6) (end 66 47.72) (width 0.4) (layer "F.Cu") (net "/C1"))
 (segment (start 68.765 44.4275) (end 68.765 45.855) (width 0.4) (layer "F.Cu") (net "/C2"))
 (segment (start 66.52 48.1) (end 66.52 49) (width 0.4) (layer "F.Cu") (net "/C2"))
 (segment (start 68.765 45.855) (end 66.52 48.1) (width 0.4) (layer "F.Cu") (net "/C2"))
 (segment (start 69.82 49) (end 69.06 49) (width 0.4) (layer "F.Cu") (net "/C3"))
 (segment (start 72.015 44.4275) (end 72.015 46.805) (width 0.4) (layer "F.Cu") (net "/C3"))
 (segment (start 72.015 46.805) (end 69.82 49) (width 0.4) (layer "F.Cu") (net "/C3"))
 (segment (start 68.765 48.805) (end 68.96 49) (width 0.4) (layer "F.Cu") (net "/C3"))
 (segment (start 72.015 48.485) (end 71.5 49) (width 0.4) (layer "F.Cu") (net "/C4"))
 (segment (start 72.665 47.935) (end 71.6 49) (width 0.4) (layer "F.Cu") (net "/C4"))
 (segment (start 72.665 44.4275) (end 72.665 47.935) (width 0.4) (layer "F.Cu") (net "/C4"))
 (segment (start 75.27 37.65) (end 74.2175 38.7025) (width 0.4) (layer "F.Cu") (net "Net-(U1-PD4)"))
 (segment (start 76.492205 37.65) (end 75.27 37.65) (width 0.4) (layer "F.Cu") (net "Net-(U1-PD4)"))
 (segment (start 74.2175 38.7025) (end 72.665 38.7025) (width 0.4) (layer "F.Cu") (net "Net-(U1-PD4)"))
 (via (at 76.492205 37.65) (size 1.9) (drill 0.9) (layers "F.Cu" "B.Cu") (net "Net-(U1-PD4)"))
 (segment (start 76.442205 37.7) (end 76.492205 37.65) (width 0.2) (layer "B.Cu") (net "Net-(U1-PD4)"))
 (segment (start 73.92 37.7) (end 76.442205 37.7) (width 0.2) (layer "B.Cu") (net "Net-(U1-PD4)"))
 (segment (start 71.365 37.905122) (end 69.859878 36.4) (width 0.4) (layer "F.Cu") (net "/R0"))
 (segment (start 71.365 38.7025) (end 71.365 37.905122) (width 0.4) (layer "F.Cu") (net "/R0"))
 (segment (start 57.87 36.4) (end 57.82 36.35) (width 0.4) (layer "F.Cu") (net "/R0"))
 (segment (start 69.859878 36.4) (end 57.87 36.4) (width 0.4) (layer "F.Cu") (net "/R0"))
 (segment (start 58.63 38.89) (end 57.82 38.89) (width 0.4) (layer "F.Cu") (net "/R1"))
 (segment (start 69.52 37.3) (end 60.22 37.3) (width 0.4) (layer "F.Cu") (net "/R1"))
 (segment (start 70.065 38.7025) (end 70.065 37.845) (width 0.4) (layer "F.Cu") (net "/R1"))
 (segment (start 60.22 37.3) (end 58.63 38.89) (width 0.4) (layer "F.Cu") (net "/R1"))
 (segment (start 70.065 37.845) (end 69.52 37.3) (width 0.4) (layer "F.Cu") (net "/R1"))
 (segment (start 69.415 38.7025) (end 69.415 40.380122) (width 0.4) (layer "F.Cu") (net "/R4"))
 (segment (start 63.8 45.8) (end 62.9 45.8) (width 0.4) (layer "F.Cu") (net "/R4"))
 (segment (start 62.9 45.8) (end 62.5 46.2) (width 0.4) (layer "F.Cu") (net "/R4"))
 (segment (start 64.65 44.95) (end 63.8 45.8) (width 0.4) (layer "F.Cu") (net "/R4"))
 (segment (start 65.074594 44.95) (end 64.65 44.95) (width 0.4) (layer "F.Cu") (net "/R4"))
 (segment (start 58.13 46.2) (end 57.82 46.51) (width 0.4) (layer "F.Cu") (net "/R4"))
 (segment (start 62.5 46.2) (end 58.13 46.2) (width 0.4) (layer "F.Cu") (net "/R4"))
 (segment (start 65.865405 44.159189) (end 65.074594 44.95) (width 0.4) (layer "F.Cu") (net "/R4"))
 (segment (start 65.865405 43.929717) (end 65.865405 44.159189) (width 0.4) (layer "F.Cu") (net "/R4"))
 (segment (start 69.415 40.380122) (end 65.865405 43.929717) (width 0.4) (layer "F.Cu") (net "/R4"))
 (segment (start 63.02 44.075) (end 61.895 45.2) (width 0.4) (layer "F.Cu") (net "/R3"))
 (segment (start 63.02 43.1) (end 63.02 44.075) (width 0.4) (layer "F.Cu") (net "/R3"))
 (segment (start 65.563406 42.25) (end 63.87 42.25) (width 0.4) (layer "F.Cu") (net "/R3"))
 (segment (start 59.05 45.2) (end 57.82 43.97) (width 0.4) (layer "F.Cu") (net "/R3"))
 (segment (start 68.115 39.698406) (end 65.563406 42.25) (width 0.4) (layer "F.Cu") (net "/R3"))
 (segment (start 68.115 38.7025) (end 68.115 39.698406) (width 0.4) (layer "F.Cu") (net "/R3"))
 (segment (start 63.87 42.25) (end 63.02 43.1) (width 0.4) (layer "F.Cu") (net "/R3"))
 (segment (start 61.895 45.2) (end 59.05 45.2) (width 0.4) (layer "F.Cu") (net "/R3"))
 (segment (start 61.149733 38.7025) (end 58.422233 41.43) (width 0.4) (layer "F.Cu") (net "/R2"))
 (segment (start 66.815 38.7025) (end 61.149733 38.7025) (width 0.4) (layer "F.Cu") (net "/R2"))
 (segment (start 58.422233 41.43) (end 57.82 41.43) (width 0.4) (layer "F.Cu") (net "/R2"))
 (segment (start 62.7 46.8) (end 62.2 47.3) (width 0.4) (layer "F.Cu") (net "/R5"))
 (segment (start 59.57 47.3) (end 57.82 49.05) (width 0.4) (layer "F.Cu") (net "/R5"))
 (segment (start 64.4425 46.8) (end 62.7 46.8) (width 0.4) (layer "F.Cu") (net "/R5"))
 (segment (start 62.2 47.3) (end 59.57 47.3) (width 0.4) (layer "F.Cu") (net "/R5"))
 (segment (start 66.815 44.4275) (end 64.4425 46.8) (width 0.4) (layer "F.Cu") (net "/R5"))
 (segment (start 71.365 44.4275) (end 71.365 45.255) (width 0.4) (layer "F.Cu") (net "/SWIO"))
 (segment (start 71.365 45.255) (end 69.92 46.7) (width 0.4) (layer "F.Cu") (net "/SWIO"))
 (via (at 69.92 46.7) (size 1.9) (drill 0.9) (layers "F.Cu" "B.Cu") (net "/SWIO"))
 (segment (start 66.72 46.7) (end 66.42 46.4) (width 0.4) (layer "B.Cu") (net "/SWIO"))
 (segment (start 69.92 46.7) (end 66.72 46.7) (width 0.4) (layer "B.Cu") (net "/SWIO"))
 (segment (start 72.12 41.4125) (end 72.77 40.7625) (width 0.4) (layer "B.Cu") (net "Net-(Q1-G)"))
 (segment (start 71.92 39.9125) (end 72.77 40.7625) (width 0.4) (layer "B.Cu") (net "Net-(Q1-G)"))
 (segment (start 71.92 37.7) (end 71.92 39.9125) (width 0.4) (layer "B.Cu") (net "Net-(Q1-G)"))
 (segment (start 72.12 43.5) (end 72.12 41.4125) (width 0.4) (layer "B.Cu") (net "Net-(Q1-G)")))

